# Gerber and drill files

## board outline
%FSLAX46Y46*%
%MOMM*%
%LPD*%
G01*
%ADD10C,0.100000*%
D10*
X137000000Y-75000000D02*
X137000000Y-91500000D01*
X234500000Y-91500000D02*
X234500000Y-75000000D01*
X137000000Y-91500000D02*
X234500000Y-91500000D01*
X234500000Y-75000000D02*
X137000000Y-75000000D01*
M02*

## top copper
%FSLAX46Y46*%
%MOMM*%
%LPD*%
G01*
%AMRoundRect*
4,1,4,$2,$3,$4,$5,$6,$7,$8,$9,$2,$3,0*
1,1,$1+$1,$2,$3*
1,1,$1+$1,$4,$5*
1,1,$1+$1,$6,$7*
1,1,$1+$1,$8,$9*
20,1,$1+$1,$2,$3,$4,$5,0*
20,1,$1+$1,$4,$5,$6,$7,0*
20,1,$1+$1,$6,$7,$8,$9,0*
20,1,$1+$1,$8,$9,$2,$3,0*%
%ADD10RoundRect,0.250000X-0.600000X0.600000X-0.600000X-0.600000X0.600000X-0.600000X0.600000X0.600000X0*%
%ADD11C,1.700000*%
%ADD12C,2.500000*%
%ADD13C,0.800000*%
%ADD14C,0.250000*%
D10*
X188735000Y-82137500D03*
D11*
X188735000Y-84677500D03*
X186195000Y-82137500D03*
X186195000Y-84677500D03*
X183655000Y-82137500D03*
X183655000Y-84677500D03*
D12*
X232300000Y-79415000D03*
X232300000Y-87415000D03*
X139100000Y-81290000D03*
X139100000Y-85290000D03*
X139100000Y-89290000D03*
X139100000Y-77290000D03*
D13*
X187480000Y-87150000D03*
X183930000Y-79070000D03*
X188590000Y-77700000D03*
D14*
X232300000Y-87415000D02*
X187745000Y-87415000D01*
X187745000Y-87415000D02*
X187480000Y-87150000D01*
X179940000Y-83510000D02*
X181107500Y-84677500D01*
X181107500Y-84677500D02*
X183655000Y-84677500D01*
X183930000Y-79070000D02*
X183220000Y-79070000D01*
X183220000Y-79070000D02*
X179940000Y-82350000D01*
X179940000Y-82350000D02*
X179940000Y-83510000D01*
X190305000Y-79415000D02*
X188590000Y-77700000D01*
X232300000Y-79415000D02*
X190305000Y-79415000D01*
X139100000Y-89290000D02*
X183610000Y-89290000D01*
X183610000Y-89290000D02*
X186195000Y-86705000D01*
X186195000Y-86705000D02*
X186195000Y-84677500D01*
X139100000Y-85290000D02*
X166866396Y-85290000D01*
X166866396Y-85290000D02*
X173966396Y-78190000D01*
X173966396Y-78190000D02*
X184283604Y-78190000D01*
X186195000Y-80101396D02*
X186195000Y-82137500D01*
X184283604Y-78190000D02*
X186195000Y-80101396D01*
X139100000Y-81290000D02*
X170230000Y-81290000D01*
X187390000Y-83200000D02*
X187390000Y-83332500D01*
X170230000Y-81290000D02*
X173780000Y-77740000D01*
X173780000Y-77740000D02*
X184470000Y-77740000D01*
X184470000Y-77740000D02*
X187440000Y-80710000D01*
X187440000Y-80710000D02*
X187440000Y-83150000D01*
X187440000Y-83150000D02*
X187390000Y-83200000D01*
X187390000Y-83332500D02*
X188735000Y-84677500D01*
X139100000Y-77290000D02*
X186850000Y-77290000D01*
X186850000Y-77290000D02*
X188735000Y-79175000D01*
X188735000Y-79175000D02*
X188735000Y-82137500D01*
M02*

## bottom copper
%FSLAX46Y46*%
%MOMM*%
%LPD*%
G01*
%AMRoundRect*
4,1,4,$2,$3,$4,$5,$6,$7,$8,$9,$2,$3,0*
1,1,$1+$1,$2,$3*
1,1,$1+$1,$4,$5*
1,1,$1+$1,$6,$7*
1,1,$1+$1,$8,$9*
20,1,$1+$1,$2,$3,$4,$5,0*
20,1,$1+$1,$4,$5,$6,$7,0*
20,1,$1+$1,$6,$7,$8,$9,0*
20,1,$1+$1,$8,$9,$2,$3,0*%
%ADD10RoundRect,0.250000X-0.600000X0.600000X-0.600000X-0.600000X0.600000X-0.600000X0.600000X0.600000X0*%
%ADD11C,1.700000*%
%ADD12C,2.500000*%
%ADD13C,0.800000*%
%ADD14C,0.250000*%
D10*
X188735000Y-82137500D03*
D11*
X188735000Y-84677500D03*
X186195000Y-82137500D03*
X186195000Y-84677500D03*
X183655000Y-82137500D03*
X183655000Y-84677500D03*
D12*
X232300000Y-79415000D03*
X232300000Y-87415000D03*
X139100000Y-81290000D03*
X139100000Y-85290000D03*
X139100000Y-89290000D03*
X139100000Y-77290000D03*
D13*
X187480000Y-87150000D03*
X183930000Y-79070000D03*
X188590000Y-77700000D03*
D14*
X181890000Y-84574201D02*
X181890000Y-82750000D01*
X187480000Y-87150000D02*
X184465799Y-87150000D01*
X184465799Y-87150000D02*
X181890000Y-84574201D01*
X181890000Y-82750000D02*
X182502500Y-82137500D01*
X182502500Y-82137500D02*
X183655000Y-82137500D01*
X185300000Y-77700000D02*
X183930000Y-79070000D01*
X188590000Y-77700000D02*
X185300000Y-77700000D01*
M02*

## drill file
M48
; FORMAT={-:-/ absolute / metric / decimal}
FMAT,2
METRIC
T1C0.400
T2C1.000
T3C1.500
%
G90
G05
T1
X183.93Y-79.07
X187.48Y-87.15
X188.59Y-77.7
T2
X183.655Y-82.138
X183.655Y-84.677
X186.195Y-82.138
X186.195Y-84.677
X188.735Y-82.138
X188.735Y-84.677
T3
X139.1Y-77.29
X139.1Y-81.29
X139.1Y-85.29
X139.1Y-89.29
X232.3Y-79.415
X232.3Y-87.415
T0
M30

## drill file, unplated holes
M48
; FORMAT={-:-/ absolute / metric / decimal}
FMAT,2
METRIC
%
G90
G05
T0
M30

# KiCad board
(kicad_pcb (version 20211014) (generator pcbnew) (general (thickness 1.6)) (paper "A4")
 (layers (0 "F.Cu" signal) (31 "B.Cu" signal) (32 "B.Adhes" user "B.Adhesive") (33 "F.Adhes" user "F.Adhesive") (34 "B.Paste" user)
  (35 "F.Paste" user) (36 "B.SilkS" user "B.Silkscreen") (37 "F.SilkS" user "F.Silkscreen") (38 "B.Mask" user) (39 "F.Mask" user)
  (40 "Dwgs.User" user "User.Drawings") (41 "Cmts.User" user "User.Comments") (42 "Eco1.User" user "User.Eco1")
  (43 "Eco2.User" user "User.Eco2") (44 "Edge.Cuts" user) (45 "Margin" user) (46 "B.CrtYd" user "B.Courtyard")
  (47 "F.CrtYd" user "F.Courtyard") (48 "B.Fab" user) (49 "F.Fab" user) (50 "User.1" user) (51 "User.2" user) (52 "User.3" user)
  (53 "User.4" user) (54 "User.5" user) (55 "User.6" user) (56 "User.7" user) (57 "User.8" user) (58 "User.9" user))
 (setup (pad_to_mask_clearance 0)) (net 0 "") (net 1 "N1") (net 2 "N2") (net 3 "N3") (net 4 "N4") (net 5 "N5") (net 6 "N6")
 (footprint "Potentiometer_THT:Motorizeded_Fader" (layer "F.Cu") (at 232.3 83.415)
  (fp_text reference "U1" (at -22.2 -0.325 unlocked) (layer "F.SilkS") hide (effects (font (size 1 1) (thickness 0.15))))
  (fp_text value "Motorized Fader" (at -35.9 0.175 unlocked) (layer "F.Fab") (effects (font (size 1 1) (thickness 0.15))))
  (pad "1" thru_hole circle (at -93.2 -6.125 180) (size 2.5 2.5) (drill 1.5) (layers *.Cu *.Mask) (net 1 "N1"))
  (pad "2" thru_hole circle (at -93.2 5.875 180) (size 2.5 2.5) (drill 1.5) (layers *.Cu *.Mask) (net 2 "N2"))
  (pad "3" thru_hole circle (at -93.2 1.875 180) (size 2.5 2.5) (drill 1.5) (layers *.Cu *.Mask) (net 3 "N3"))
  (pad "4" thru_hole circle (at -93.2 -2.125 180) (size 2.5 2.5) (drill 1.5) (layers *.Cu *.Mask) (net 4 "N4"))
  (pad "5" thru_hole circle (at 0 4) (size 2.5 2.5) (drill 1.5) (layers *.Cu *.Mask) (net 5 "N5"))
  (pad "6" thru_hole circle (at 0 -4) (size 2.5 2.5) (drill 1.5) (layers *.Cu *.Mask) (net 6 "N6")))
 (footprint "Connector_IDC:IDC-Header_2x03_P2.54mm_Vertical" (layer "F.Cu") (at 188.735 82.1375 -90)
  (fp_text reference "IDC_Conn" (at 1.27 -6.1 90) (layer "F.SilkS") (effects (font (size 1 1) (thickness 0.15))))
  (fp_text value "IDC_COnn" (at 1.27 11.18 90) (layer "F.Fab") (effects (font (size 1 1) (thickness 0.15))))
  (pad "1" thru_hole roundrect (at 0 0 270) (size 1.7 1.7) (drill 1) (layers *.Cu *.Mask) (roundrect_rratio 0.1470588235) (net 1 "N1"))
  (pad "2" thru_hole circle (at 2.54 0 270) (size 1.7 1.7) (drill 1) (layers *.Cu *.Mask) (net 4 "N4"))
  (pad "3" thru_hole circle (at 0 2.54 270) (size 1.7 1.7) (drill 1) (layers *.Cu *.Mask) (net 3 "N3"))
  (pad "4" thru_hole circle (at 2.54 2.54 270) (size 1.7 1.7) (drill 1) (layers *.Cu *.Mask) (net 2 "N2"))
  (pad "5" thru_hole circle (at 0 5.08 270) (size 1.7 1.7) (drill 1) (layers *.Cu *.Mask) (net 5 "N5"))
  (pad "6" thru_hole circle (at 2.54 5.08 270) (size 1.7 1.7) (drill 1) (layers *.Cu *.Mask) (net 6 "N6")))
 (gr_line (start 137 75) (end 137 91.5) (layer "Edge.Cuts") (width 0.1))
 (gr_line (start 234.5 91.5) (end 234.5 75) (layer "Edge.Cuts") (width 0.1))
 (gr_line (start 137 91.5) (end 234.5 91.5) (layer "Edge.Cuts") (width 0.1))
 (gr_line (start 234.5 75) (end 137 75) (layer "Edge.Cuts") (width 0.1))
 (segment (start 188.735 79.175) (end 188.735 82.1375) (width 0.25) (layer "F.Cu") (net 1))
 (segment (start 186.85 77.29) (end 188.735 79.175) (width 0.25) (layer "F.Cu") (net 1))
 (segment (start 139.1 77.29) (end 186.85 77.29) (width 0.25) (layer "F.Cu") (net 1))
 (segment (start 187.39 83.3325) (end 188.735 84.6775) (width 0.25) (layer "F.Cu") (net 4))
 (segment (start 187.44 83.15) (end 187.39 83.2) (width 0.25) (layer "F.Cu") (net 4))
 (segment (start 187.44 80.71) (end 187.44 83.15) (width 0.25) (layer "F.Cu") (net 4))
 (segment (start 170.23 81.29) (end 173.78 77.74) (width 0.25) (layer "F.Cu") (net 4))
 (segment (start 184.47 77.74) (end 187.44 80.71) (width 0.25) (layer "F.Cu") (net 4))
 (segment (start 187.39 83.2) (end 187.39 83.3325) (width 0.25) (layer "F.Cu") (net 4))
 (segment (start 139.1 81.29) (end 170.23 81.29) (width 0.25) (layer "F.Cu") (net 4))
 (segment (start 173.78 77.74) (end 184.47 77.74) (width 0.25) (layer "F.Cu") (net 4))
 (segment (start 173.966396 78.19) (end 184.283604 78.19) (width 0.25) (layer "F.Cu") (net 3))
 (segment (start 184.283604 78.19) (end 186.195 80.101396) (width 0.25) (layer "F.Cu") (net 3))
 (segment (start 139.1 85.29) (end 166.866396 85.29) (width 0.25) (layer "F.Cu") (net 3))
 (segment (start 186.195 80.101396) (end 186.195 82.1375) (width 0.25) (layer "F.Cu") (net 3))
 (segment (start 166.866396 85.29) (end 173.966396 78.19) (width 0.25) (layer "F.Cu") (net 3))
 (segment (start 183.61 89.29) (end 186.195 86.705) (width 0.25) (layer "F.Cu") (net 2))
 (segment (start 139.1 89.29) (end 183.61 89.29) (width 0.25) (layer "F.Cu") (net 2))
 (segment (start 186.195 86.705) (end 186.195 84.6775) (width 0.25) (layer "F.Cu") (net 2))
 (segment (start 187.745 87.415) (end 187.48 87.15) (width 0.25) (layer "F.Cu") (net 5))
 (segment (start 232.3 87.415) (end 187.745 87.415) (width 0.25) (layer "F.Cu") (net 5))
 (via (at 187.48 87.15) (size 0.8) (drill 0.4) (layers "F.Cu" "B.Cu") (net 5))
 (segment (start 182.5025 82.1375) (end 183.655 82.1375) (width 0.25) (layer "B.Cu") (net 5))
 (segment (start 184.465799 87.15) (end 181.89 84.574201) (width 0.25) (layer "B.Cu") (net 5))
 (segment (start 187.48 87.15) (end 184.465799 87.15) (width 0.25) (layer "B.Cu") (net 5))
 (segment (start 181.89 84.574201) (end 181.89 82.75) (width 0.25) (layer "B.Cu") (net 5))
 (segment (start 181.89 82.75) (end 182.5025 82.1375) (width 0.25) (layer "B.Cu") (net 5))
 (segment (start 183.93 79.07) (end 183.22 79.07) (width 0.25) (layer "F.Cu") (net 6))
 (segment (start 232.3 79.415) (end 190.305 79.415) (width 0.25) (layer "F.Cu") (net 6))
 (segment (start 183.22 79.07) (end 179.94 82.35) (width 0.25) (layer "F.Cu") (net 6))
 (segment (start 190.305 79.415) (end 188.59 77.7) (width 0.25) (layer "F.Cu") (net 6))
 (segment (start 179.94 82.35) (end 179.94 83.51) (width 0.25) (layer "F.Cu") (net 6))
 (segment (start 181.1075 84.6775) (end 183.655 84.6775) (width 0.25) (layer "F.Cu") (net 6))
 (segment (start 179.94 83.51) (end 181.1075 84.6775) (width 0.25) (layer "F.Cu") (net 6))
 (via (at 183.93 79.07) (size 0.8) (drill 0.4) (layers "F.Cu" "B.Cu") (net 6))
 (via (at 188.59 77.7) (size 0.8) (drill 0.4) (layers "F.Cu" "B.Cu") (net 6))
 (segment (start 185.3 77.7) (end 183.93 79.07) (width 0.25) (layer "B.Cu") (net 6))
 (segment (start 188.59 77.7) (end 185.3 77.7) (width 0.25) (layer "B.Cu") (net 6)))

